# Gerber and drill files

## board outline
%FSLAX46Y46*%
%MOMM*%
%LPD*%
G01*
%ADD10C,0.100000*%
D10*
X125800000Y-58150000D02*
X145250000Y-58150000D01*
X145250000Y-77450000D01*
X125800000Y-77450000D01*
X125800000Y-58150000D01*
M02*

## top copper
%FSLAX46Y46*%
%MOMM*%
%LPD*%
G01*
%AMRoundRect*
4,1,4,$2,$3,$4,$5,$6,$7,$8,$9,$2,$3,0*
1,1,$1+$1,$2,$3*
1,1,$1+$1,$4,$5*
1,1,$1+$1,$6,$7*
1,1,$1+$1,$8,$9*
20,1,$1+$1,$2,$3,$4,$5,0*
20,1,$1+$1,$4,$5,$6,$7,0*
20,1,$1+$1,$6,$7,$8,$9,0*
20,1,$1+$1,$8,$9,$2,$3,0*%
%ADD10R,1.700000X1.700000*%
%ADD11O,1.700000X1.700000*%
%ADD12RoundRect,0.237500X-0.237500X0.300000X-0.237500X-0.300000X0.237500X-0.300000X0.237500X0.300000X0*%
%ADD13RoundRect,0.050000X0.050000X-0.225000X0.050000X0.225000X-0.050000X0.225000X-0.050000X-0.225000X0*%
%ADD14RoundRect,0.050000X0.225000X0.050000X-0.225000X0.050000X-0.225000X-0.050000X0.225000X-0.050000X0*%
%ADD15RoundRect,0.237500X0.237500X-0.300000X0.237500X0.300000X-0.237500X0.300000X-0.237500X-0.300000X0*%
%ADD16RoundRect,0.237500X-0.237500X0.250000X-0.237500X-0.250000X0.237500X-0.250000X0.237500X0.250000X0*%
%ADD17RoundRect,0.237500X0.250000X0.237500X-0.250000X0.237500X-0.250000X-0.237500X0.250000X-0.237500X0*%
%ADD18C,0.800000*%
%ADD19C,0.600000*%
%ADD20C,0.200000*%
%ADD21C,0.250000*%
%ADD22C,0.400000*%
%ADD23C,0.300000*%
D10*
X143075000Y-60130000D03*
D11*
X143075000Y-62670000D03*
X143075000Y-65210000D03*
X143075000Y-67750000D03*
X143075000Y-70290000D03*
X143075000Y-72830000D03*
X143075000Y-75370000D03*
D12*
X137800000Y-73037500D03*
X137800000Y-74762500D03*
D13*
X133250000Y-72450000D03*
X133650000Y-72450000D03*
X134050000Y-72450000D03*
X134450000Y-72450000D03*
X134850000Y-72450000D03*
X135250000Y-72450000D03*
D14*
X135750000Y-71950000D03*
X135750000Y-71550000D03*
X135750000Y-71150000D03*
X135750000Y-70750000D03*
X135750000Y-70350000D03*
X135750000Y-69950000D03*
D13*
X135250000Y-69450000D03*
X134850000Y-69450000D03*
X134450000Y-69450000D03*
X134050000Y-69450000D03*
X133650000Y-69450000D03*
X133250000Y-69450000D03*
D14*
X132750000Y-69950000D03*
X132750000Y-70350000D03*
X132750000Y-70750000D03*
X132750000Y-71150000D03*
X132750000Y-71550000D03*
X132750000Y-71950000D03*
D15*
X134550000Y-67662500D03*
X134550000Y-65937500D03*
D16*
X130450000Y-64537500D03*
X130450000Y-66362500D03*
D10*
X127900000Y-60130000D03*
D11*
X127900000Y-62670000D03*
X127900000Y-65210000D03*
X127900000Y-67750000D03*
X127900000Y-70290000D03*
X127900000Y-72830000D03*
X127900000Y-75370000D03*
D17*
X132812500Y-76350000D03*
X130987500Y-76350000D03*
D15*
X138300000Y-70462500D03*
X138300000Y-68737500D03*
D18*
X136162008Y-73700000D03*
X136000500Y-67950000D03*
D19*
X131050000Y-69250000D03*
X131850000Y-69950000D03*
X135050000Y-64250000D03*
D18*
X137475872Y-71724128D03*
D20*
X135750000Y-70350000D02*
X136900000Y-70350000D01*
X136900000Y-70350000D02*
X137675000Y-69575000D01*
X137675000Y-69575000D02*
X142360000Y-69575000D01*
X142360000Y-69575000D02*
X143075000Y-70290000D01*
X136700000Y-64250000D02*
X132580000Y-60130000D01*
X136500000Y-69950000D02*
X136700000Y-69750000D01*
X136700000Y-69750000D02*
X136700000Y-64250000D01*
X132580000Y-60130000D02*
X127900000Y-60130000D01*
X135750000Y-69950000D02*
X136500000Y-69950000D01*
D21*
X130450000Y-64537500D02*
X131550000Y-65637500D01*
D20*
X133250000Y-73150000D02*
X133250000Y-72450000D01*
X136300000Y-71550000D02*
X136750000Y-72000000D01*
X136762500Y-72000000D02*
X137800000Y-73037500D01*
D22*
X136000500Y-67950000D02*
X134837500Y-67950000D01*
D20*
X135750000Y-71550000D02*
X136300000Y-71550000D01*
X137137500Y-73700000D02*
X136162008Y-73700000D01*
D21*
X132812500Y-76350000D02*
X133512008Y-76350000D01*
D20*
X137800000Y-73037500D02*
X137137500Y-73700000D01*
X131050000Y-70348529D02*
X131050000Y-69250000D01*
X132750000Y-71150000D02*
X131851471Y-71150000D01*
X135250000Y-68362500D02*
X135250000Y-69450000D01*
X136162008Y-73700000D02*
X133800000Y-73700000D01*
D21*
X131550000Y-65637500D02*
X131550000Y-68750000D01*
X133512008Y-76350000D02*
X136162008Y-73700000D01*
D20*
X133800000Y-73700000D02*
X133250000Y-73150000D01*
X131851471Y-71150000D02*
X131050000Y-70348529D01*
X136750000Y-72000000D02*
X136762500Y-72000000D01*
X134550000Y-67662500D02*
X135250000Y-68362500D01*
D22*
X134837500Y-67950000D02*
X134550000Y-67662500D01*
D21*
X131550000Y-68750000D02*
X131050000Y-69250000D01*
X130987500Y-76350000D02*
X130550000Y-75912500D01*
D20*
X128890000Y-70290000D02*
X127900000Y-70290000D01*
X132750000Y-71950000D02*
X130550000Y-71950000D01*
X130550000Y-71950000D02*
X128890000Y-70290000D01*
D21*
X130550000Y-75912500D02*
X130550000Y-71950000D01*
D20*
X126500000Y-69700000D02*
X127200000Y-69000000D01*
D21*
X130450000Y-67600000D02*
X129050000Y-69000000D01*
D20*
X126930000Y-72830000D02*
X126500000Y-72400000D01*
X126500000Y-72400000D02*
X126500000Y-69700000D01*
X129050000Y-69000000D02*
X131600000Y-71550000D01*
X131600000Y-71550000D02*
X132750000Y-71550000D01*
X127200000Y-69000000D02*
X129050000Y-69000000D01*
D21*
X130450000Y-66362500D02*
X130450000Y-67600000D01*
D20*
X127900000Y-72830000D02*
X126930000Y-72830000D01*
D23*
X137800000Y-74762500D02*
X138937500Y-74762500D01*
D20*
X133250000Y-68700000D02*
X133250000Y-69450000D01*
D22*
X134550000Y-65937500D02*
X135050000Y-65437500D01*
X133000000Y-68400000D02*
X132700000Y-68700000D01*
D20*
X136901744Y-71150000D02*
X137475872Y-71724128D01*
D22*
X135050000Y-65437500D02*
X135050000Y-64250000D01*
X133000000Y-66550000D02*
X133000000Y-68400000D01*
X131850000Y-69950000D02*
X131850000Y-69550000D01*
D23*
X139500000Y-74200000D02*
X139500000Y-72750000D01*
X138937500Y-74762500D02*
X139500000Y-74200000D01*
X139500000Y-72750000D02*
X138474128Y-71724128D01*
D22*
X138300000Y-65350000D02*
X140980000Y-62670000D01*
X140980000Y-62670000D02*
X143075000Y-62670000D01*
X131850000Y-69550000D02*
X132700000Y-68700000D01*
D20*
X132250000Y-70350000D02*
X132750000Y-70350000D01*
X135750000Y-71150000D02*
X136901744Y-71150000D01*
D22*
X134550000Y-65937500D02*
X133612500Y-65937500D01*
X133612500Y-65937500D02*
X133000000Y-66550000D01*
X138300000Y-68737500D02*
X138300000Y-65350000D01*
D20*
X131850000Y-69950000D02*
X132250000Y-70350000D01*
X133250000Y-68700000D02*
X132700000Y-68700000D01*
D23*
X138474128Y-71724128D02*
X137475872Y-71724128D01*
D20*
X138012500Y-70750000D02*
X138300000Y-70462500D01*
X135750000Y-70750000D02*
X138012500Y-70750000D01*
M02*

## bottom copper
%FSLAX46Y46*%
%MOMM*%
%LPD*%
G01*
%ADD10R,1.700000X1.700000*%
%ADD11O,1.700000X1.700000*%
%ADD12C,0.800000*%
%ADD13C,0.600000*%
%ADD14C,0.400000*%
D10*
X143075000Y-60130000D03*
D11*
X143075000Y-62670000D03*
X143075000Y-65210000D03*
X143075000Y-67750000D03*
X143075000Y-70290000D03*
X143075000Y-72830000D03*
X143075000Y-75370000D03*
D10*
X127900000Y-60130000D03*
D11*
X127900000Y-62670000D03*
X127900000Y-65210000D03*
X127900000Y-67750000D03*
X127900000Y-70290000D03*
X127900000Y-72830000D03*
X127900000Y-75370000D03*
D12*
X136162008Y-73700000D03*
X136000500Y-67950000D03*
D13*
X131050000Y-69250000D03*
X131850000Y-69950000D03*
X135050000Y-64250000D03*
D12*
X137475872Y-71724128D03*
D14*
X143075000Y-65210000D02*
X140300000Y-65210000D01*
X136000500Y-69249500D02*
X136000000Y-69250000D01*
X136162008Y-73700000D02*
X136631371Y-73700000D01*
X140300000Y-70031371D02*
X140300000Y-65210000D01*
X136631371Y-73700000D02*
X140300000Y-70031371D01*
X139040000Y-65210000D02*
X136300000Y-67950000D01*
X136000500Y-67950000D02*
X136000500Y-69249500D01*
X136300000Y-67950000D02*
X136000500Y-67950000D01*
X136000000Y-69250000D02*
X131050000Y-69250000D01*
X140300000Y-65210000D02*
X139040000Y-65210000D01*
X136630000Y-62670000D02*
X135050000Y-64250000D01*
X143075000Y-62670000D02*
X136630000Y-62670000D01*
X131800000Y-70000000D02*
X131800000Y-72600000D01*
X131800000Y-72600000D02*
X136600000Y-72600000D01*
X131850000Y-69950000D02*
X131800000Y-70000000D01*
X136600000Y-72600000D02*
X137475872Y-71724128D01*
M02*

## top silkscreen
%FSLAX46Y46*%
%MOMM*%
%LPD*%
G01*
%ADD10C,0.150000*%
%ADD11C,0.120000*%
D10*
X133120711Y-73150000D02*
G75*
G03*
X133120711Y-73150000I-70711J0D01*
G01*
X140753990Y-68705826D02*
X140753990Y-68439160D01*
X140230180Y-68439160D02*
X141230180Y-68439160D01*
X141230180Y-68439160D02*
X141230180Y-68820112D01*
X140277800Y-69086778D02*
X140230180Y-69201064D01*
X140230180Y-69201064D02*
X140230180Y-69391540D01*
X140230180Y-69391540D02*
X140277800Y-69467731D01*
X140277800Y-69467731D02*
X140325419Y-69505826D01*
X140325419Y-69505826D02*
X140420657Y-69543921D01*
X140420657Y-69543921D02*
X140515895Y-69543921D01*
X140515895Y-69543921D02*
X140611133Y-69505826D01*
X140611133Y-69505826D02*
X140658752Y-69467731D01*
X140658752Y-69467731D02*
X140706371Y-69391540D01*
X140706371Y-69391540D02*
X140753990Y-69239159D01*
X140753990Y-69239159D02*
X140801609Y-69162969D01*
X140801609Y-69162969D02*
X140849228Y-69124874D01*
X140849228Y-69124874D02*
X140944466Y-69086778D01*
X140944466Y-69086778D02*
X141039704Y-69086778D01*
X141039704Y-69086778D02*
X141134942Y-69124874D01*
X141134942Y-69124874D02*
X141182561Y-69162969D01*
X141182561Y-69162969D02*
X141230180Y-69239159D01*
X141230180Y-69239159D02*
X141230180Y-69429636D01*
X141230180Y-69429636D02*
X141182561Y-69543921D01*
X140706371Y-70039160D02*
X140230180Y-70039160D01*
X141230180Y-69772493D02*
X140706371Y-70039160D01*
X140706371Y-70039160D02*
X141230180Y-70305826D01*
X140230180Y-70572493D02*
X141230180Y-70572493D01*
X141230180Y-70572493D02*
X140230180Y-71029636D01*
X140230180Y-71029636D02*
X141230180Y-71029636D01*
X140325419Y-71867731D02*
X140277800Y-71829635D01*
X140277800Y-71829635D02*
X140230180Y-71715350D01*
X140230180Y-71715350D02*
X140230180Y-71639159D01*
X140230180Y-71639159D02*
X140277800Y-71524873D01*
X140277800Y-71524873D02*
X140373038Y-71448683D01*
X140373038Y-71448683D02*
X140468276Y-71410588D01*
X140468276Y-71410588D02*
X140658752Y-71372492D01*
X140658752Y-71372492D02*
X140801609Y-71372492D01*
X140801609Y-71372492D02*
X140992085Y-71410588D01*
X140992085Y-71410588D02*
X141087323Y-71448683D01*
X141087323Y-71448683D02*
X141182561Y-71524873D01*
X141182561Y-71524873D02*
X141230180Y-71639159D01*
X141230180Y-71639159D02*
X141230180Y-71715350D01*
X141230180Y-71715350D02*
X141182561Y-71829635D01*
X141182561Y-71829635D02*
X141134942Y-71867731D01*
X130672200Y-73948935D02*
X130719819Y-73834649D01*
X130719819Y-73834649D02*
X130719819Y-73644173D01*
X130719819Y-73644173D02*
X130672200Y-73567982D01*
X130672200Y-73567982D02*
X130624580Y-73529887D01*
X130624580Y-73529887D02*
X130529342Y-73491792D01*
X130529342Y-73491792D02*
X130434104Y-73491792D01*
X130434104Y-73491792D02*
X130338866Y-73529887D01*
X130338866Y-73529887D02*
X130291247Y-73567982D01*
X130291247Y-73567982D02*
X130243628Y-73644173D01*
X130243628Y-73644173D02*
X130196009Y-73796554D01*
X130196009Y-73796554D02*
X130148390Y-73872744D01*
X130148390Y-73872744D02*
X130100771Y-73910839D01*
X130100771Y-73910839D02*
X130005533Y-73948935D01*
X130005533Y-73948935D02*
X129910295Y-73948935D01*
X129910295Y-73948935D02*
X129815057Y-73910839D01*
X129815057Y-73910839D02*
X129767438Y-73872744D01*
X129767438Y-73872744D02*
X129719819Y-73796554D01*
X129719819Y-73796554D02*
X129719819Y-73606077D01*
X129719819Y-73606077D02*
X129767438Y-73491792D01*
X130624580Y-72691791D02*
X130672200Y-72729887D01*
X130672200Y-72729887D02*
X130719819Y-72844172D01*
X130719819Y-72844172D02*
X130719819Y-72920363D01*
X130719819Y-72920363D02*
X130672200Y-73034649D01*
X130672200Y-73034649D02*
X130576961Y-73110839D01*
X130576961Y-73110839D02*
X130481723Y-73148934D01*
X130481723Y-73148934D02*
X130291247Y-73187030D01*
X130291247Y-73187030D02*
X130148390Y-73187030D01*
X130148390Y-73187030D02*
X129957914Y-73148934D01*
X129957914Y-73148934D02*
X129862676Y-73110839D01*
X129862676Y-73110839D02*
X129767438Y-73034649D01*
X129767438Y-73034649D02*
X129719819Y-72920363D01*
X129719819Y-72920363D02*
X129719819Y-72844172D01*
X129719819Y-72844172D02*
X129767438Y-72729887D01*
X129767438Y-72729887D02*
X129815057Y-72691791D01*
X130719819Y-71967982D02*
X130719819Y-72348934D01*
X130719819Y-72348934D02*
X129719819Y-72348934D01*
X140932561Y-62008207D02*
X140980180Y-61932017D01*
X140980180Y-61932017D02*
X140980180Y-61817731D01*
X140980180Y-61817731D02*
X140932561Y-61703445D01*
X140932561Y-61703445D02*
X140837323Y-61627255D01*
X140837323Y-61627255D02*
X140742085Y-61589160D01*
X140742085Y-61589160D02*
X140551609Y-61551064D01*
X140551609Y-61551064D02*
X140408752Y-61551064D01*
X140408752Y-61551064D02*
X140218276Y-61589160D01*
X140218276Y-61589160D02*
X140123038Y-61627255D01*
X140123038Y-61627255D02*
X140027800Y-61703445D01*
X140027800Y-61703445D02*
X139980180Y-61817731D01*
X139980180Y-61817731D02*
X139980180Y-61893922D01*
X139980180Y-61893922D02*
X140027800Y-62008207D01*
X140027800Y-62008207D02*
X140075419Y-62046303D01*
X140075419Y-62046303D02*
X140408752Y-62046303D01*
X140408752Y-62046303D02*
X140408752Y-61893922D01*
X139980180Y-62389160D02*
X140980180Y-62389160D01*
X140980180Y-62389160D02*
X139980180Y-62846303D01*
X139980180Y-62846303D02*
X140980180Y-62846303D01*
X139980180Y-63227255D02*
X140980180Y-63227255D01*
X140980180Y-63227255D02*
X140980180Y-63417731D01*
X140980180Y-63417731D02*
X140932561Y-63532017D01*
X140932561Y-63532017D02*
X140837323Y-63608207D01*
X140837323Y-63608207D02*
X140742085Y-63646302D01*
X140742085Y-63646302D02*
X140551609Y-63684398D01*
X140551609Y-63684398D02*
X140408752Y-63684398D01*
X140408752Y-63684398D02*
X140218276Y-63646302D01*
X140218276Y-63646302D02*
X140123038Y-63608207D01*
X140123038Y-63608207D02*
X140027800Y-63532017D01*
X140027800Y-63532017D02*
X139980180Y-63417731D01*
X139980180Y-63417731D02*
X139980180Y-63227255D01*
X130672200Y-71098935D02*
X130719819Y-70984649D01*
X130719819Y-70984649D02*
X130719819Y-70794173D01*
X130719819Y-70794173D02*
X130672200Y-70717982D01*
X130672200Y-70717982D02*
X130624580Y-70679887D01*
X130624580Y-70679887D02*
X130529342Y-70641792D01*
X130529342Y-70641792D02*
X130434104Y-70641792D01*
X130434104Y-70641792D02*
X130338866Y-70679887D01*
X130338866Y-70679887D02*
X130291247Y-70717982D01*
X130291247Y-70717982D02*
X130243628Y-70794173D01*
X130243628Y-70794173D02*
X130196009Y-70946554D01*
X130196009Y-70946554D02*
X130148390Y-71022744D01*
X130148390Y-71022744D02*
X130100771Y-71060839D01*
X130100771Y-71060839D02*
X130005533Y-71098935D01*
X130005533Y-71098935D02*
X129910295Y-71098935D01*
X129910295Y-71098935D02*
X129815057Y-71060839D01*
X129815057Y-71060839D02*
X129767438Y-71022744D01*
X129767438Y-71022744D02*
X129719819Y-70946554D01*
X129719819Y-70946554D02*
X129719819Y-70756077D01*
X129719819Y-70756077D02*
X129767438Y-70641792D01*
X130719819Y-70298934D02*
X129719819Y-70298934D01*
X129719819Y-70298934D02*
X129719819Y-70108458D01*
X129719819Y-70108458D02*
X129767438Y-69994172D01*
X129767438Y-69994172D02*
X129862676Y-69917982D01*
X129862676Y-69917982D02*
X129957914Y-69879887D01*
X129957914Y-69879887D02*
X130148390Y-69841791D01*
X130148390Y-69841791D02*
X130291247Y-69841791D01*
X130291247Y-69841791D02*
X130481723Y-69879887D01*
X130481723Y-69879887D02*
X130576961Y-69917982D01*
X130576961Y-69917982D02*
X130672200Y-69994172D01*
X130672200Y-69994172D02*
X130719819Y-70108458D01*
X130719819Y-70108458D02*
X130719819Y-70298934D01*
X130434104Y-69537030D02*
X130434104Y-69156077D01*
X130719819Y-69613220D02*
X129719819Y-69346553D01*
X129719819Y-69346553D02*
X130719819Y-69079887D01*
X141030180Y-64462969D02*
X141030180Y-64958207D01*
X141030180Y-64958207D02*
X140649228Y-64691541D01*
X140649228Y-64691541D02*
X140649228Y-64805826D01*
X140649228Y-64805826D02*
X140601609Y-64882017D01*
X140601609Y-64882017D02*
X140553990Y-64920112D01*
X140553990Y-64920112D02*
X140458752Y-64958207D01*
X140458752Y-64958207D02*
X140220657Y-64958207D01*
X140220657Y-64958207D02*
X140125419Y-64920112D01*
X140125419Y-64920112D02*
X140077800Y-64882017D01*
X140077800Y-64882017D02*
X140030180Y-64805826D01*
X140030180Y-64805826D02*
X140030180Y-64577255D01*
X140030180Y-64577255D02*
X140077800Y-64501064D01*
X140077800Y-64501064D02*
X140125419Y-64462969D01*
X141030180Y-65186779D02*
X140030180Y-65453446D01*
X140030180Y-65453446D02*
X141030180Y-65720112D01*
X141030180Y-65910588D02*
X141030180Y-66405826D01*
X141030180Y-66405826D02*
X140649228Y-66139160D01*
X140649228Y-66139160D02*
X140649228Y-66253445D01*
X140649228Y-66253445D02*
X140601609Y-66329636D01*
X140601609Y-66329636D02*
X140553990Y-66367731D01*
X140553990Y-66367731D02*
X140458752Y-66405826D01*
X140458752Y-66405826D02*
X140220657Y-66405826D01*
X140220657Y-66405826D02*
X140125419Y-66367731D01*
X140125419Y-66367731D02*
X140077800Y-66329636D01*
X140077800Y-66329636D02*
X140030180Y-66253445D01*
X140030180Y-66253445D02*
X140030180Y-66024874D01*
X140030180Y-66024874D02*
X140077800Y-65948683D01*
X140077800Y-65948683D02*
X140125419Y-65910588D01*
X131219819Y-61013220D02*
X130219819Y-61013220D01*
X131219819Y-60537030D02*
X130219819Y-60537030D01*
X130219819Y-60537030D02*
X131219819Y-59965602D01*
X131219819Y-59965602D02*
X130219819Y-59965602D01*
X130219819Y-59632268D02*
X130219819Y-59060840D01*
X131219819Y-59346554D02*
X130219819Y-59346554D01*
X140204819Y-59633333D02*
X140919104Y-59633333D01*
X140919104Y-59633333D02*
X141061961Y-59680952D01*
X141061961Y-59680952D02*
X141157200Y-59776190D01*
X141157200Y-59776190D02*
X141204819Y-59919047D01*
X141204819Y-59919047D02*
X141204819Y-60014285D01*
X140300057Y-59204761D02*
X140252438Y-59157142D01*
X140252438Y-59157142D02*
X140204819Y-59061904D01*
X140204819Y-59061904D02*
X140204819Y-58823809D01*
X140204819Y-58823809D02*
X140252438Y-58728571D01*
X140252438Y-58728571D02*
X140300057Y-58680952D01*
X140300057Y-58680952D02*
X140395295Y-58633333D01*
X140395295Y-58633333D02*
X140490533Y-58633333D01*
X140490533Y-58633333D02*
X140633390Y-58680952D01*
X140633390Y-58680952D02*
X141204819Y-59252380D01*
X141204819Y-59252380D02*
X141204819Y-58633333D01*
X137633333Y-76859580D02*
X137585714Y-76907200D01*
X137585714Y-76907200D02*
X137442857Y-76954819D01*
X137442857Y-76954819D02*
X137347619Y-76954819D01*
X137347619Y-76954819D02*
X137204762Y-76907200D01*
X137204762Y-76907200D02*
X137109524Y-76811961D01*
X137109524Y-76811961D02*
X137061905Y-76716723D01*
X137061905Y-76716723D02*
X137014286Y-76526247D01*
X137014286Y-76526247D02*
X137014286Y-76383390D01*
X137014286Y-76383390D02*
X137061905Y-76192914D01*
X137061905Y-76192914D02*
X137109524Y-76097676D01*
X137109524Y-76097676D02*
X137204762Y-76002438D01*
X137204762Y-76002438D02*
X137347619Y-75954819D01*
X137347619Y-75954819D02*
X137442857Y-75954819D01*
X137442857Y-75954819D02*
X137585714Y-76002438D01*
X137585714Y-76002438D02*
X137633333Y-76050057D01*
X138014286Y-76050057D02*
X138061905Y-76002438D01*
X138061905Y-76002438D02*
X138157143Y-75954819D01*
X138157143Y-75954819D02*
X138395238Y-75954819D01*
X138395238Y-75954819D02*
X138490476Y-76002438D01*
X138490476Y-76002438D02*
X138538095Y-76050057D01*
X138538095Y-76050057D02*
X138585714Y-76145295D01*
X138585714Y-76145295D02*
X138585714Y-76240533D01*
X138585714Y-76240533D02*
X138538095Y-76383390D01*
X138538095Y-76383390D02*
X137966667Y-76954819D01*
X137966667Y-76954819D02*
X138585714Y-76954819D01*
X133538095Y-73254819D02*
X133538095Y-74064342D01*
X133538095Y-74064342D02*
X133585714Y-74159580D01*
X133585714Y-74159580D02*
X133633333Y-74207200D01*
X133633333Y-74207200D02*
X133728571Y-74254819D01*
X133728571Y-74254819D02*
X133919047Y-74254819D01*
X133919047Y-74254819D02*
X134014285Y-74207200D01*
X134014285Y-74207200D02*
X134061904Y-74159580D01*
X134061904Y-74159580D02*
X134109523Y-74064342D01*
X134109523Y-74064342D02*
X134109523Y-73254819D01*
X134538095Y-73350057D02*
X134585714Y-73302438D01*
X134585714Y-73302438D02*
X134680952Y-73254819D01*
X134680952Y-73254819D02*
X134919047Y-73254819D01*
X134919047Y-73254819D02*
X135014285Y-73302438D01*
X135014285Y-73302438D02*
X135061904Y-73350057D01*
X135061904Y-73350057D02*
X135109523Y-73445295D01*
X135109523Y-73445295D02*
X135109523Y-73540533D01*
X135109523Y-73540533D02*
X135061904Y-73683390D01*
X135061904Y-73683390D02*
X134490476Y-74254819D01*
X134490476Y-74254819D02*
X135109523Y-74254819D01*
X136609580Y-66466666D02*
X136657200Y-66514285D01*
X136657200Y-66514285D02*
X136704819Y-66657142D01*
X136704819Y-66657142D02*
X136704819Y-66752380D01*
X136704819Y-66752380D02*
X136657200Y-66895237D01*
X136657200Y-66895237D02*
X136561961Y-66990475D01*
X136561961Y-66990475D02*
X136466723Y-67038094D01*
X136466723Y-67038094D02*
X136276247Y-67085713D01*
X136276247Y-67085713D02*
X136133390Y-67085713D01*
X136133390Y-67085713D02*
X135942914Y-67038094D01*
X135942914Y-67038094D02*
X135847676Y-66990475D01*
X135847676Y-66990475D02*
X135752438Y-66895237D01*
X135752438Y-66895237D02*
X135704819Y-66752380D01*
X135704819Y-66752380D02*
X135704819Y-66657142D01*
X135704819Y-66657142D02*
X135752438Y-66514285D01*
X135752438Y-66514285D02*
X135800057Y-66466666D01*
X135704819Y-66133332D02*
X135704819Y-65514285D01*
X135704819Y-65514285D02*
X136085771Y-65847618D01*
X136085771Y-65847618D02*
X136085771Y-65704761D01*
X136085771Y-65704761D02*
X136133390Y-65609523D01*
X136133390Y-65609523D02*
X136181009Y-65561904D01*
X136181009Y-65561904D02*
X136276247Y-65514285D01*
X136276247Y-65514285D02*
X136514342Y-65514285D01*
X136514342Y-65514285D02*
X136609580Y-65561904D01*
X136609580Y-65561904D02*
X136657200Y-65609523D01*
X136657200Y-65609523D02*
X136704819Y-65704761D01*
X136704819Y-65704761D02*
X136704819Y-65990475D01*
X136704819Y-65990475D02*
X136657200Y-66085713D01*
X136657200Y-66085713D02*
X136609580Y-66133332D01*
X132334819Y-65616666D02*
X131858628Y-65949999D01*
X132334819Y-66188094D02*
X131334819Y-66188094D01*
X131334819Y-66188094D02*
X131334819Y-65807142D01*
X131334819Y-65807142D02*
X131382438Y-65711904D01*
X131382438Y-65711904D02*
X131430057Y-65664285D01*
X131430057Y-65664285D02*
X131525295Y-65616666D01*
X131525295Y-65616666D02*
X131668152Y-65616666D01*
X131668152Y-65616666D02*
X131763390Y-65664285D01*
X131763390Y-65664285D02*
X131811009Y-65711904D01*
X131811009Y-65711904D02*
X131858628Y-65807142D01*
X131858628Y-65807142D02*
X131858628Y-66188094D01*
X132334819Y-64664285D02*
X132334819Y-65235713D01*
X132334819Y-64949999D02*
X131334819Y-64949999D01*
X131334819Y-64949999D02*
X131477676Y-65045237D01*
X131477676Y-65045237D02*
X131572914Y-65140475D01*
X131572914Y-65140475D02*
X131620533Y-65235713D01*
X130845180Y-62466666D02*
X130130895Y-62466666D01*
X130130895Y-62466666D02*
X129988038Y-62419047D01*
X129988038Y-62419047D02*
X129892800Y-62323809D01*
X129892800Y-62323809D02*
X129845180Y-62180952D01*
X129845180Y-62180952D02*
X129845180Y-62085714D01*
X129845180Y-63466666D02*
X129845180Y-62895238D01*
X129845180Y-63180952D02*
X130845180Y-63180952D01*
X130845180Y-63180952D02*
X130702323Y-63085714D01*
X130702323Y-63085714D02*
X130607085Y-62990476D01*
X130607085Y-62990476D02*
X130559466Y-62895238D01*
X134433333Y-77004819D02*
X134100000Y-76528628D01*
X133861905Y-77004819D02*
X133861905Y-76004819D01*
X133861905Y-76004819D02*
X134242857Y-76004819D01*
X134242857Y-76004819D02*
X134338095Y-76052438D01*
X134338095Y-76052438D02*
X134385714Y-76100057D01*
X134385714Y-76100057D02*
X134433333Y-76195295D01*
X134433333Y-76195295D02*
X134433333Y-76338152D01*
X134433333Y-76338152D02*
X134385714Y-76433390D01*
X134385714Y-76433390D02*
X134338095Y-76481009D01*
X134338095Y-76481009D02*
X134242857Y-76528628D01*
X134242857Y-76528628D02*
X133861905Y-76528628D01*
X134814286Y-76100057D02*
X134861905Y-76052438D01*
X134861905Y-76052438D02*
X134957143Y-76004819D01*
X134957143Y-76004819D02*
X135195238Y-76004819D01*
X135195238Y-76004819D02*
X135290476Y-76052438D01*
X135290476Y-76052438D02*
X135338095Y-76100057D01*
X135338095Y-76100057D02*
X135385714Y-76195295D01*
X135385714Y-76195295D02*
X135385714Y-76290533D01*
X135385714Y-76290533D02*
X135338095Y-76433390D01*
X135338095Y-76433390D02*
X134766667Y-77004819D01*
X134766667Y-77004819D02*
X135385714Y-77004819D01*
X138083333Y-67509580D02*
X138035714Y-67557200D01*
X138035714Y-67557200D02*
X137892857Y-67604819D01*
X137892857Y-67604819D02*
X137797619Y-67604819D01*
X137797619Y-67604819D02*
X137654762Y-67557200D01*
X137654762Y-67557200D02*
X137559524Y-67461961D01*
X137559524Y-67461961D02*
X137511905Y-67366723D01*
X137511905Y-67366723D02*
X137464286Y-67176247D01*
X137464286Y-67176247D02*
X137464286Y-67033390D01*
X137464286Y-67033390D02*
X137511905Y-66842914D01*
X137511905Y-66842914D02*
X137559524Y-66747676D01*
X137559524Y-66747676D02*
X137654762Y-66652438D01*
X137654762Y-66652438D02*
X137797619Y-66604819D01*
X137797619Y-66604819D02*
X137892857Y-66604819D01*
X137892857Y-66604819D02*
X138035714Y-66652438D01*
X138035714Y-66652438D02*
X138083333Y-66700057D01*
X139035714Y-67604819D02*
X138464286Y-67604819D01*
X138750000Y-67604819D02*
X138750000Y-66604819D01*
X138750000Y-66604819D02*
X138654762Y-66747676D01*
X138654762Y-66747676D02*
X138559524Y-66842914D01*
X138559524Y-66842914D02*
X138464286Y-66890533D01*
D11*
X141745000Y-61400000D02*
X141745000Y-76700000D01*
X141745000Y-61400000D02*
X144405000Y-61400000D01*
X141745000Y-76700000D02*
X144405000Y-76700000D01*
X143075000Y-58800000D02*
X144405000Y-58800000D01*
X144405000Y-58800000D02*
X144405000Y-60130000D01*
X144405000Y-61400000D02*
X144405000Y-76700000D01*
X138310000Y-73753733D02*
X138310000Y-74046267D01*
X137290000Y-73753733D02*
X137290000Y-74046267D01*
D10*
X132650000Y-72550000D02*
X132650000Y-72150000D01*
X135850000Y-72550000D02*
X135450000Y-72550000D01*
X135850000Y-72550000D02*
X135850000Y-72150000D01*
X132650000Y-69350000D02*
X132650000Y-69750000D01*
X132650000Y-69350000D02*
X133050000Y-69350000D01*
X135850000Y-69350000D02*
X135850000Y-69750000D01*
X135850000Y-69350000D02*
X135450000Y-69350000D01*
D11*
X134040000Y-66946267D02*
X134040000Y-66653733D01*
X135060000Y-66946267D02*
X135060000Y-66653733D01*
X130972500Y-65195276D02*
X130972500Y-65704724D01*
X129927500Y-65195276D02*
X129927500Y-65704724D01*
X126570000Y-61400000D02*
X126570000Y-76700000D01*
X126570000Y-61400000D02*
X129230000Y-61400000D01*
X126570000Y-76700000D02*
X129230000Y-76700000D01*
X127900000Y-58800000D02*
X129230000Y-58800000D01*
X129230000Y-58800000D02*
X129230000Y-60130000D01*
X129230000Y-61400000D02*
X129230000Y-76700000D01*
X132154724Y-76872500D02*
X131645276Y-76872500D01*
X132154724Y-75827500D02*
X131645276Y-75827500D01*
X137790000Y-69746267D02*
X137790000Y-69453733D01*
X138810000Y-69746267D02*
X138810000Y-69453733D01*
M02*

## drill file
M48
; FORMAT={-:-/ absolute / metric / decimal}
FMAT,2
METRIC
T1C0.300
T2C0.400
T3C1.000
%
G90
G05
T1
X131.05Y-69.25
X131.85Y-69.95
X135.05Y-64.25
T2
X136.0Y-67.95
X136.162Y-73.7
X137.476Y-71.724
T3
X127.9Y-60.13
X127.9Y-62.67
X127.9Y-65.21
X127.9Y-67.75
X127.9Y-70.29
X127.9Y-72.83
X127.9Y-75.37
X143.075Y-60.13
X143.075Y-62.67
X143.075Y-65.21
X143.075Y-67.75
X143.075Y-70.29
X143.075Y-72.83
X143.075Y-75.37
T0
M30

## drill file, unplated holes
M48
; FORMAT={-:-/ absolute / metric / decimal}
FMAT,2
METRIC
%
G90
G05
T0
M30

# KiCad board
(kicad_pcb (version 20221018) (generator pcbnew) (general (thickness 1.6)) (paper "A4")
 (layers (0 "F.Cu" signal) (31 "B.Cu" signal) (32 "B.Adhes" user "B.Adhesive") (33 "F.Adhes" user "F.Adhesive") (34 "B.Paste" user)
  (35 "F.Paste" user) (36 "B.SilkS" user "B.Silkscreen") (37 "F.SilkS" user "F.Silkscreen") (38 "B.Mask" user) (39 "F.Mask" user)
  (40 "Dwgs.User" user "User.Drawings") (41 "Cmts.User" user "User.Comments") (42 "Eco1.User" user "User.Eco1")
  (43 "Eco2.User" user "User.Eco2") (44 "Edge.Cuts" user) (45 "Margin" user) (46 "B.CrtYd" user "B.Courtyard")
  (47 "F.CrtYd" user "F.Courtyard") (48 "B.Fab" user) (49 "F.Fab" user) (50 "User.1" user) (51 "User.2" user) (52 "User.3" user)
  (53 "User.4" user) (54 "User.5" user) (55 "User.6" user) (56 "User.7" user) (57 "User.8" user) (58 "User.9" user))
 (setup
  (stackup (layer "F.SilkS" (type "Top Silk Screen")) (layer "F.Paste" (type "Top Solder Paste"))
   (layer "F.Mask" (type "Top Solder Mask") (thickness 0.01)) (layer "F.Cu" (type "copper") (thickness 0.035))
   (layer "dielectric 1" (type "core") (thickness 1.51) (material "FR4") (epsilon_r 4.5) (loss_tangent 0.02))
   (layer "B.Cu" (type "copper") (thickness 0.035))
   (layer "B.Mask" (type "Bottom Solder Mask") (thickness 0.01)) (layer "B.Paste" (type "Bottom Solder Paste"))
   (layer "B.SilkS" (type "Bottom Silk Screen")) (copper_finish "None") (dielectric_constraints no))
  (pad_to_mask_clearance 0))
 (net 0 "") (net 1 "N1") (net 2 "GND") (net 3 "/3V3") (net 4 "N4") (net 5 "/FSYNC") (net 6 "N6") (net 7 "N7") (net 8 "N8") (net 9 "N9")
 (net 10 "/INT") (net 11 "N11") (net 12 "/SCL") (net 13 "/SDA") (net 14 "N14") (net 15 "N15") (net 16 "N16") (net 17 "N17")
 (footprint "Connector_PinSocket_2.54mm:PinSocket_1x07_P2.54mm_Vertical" (layer "F.Cu") (at 143.075 60.13)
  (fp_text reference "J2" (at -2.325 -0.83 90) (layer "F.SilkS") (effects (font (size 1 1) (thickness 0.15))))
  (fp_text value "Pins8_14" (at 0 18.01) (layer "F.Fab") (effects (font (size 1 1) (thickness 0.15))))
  (fp_line (start -1.33 1.27) (end -1.33 16.57) (stroke (width 0.12) (type solid)) (layer "F.SilkS"))
  (fp_line (start -1.33 1.27) (end 1.33 1.27) (stroke (width 0.12) (type solid)) (layer "F.SilkS"))
  (fp_line (start -1.33 16.57) (end 1.33 16.57) (stroke (width 0.12) (type solid)) (layer "F.SilkS"))
  (fp_line (start 0 -1.33) (end 1.33 -1.33) (stroke (width 0.12) (type solid)) (layer "F.SilkS"))
  (fp_line (start 1.33 -1.33) (end 1.33 0) (stroke (width 0.12) (type solid)) (layer "F.SilkS"))
  (fp_line (start 1.33 1.27) (end 1.33 16.57) (stroke (width 0.12) (type solid)) (layer "F.SilkS"))
  (pad "1" thru_hole rect (at 0 0) (size 1.7 1.7) (drill 1) (layers "*.Cu" "*.Mask") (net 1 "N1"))
  (pad "2" thru_hole oval (at 0 2.54) (size 1.7 1.7) (drill 1) (layers "*.Cu" "*.Mask") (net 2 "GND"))
  (pad "3" thru_hole oval (at 0 5.08) (size 1.7 1.7) (drill 1) (layers "*.Cu" "*.Mask") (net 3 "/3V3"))
  (pad "4" thru_hole oval (at 0 7.62) (size 1.7 1.7) (drill 1) (layers "*.Cu" "*.Mask") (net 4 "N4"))
  (pad "5" thru_hole oval (at 0 10.16) (size 1.7 1.7) (drill 1) (layers "*.Cu" "*.Mask") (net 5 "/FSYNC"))
  (pad "6" thru_hole oval (at 0 12.7) (size 1.7 1.7) (drill 1) (layers "*.Cu" "*.Mask") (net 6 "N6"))
  (pad "7" thru_hole oval (at 0 15.24) (size 1.7 1.7) (drill 1) (layers "*.Cu" "*.Mask") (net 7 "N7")))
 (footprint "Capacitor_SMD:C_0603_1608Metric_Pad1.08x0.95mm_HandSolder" (layer "F.Cu") (at 137.8 73.9 -90)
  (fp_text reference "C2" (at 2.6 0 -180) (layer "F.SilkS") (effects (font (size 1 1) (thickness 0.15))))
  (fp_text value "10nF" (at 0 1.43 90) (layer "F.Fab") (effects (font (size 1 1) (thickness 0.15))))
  (fp_line (start -0.146267 -0.51) (end 0.146267 -0.51) (stroke (width 0.12) (type solid)) (layer "F.SilkS"))
  (fp_line (start -0.146267 0.51) (end 0.146267 0.51) (stroke (width 0.12) (type solid)) (layer "F.SilkS"))
  (pad "1" smd roundrect (at -0.8625 0 270) (size 1.075 0.95) (layers "F.Cu" "F.Paste" "F.Mask") (roundrect_rratio 0.25) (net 3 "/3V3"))
  (pad "2" smd roundrect (at 0.8625 0 270) (size 1.075 0.95) (layers "F.Cu" "F.Paste" "F.Mask") (roundrect_rratio 0.25) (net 2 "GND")))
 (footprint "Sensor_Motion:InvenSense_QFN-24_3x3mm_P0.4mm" (layer "F.Cu") (at 134.25 70.95 90)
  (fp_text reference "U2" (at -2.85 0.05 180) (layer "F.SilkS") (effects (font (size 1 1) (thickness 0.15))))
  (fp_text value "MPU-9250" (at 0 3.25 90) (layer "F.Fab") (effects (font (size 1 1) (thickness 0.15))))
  (fp_line (start -1.6 -1.6) (end -1.2 -1.6) (stroke (width 0.15) (type solid)) (layer "F.SilkS"))
  (fp_line (start -1.6 1.6) (end -1.6 1.2) (stroke (width 0.15) (type solid)) (layer "F.SilkS"))
  (fp_line (start -1.6 1.6) (end -1.2 1.6) (stroke (width 0.15) (type solid)) (layer "F.SilkS"))
  (fp_line (start 1.6 -1.6) (end 1.2 -1.6) (stroke (width 0.15) (type solid)) (layer "F.SilkS"))
  (fp_line (start 1.6 -1.6) (end 1.6 -1.2) (stroke (width 0.15) (type solid)) (layer "F.SilkS"))
  (fp_line (start 1.6 1.6) (end 1.2 1.6) (stroke (width 0.15) (type solid)) (layer "F.SilkS"))
  (fp_line (start 1.6 1.6) (end 1.6 1.2) (stroke (width 0.15) (type solid)) (layer "F.SilkS"))
  (pad "1" smd roundrect (at -1.5 -1 90) (size 0.55 0.2) (layers "F.Cu" "F.Paste" "F.Mask") (roundrect_rratio 0.25) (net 3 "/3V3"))
  (pad "2" smd roundrect (at -1.5 -0.6 90) (size 0.55 0.2) (layers "F.Cu" "F.Paste" "F.Mask") (roundrect_rratio 0.25))
  (pad "3" smd roundrect (at -1.5 -0.2 90) (size 0.55 0.2) (layers "F.Cu" "F.Paste" "F.Mask") (roundrect_rratio 0.25))
  (pad "4" smd roundrect (at -1.5 0.2 90) (size 0.55 0.2) (layers "F.Cu" "F.Paste" "F.Mask") (roundrect_rratio 0.25))
  (pad "5" smd roundrect (at -1.5 0.6 90) (size 0.55 0.2) (layers "F.Cu" "F.Paste" "F.Mask") (roundrect_rratio 0.25))
  (pad "6" smd roundrect (at -1.5 1 90) (size 0.55 0.2) (layers "F.Cu" "F.Paste" "F.Mask") (roundrect_rratio 0.25))
  (pad "7" smd roundrect (at -1 1.5 180) (size 0.55 0.2) (layers "F.Cu" "F.Paste" "F.Mask") (roundrect_rratio 0.25) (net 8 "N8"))
  (pad "8" smd roundrect (at -0.6 1.5 180) (size 0.55 0.2) (layers "F.Cu" "F.Paste" "F.Mask") (roundrect_rratio 0.25) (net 3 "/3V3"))
  (pad "9" smd roundrect (at -0.2 1.5 180) (size 0.55 0.2) (layers "F.Cu" "F.Paste" "F.Mask") (roundrect_rratio 0.25) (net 2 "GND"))
  (pad "10" smd roundrect (at 0.2 1.5 180) (size 0.55 0.2) (layers "F.Cu" "F.Paste" "F.Mask") (roundrect_rratio 0.25) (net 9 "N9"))
  (pad "11" smd roundrect (at 0.6 1.5 180) (size 0.55 0.2) (layers "F.Cu" "F.Paste" "F.Mask") (roundrect_rratio 0.25) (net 5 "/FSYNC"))
  (pad "12" smd roundrect (at 1 1.5 180) (size 0.55 0.2) (layers "F.Cu" "F.Paste" "F.Mask") (roundrect_rratio 0.25) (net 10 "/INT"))
  (pad "13" smd roundrect (at 1.5 1 90) (size 0.55 0.2) (layers "F.Cu" "F.Paste" "F.Mask") (roundrect_rratio 0.25) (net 3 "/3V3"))
  (pad "14" smd roundrect (at 1.5 0.6 90) (size 0.55 0.2) (layers "F.Cu" "F.Paste" "F.Mask") (roundrect_rratio 0.25))
  (pad "15" smd roundrect (at 1.5 0.2 90) (size 0.55 0.2) (layers "F.Cu" "F.Paste" "F.Mask") (roundrect_rratio 0.25))
  (pad "16" smd roundrect (at 1.5 -0.2 90) (size 0.55 0.2) (layers "F.Cu" "F.Paste" "F.Mask") (roundrect_rratio 0.25))
  (pad "17" smd roundrect (at 1.5 -0.6 90) (size 0.55 0.2) (layers "F.Cu" "F.Paste" "F.Mask") (roundrect_rratio 0.25))
  (pad "18" smd roundrect (at 1.5 -1 90) (size 0.55 0.2) (layers "F.Cu" "F.Paste" "F.Mask") (roundrect_rratio 0.25) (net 2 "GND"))
  (pad "19" smd roundrect (at 1 -1.5 180) (size 0.55 0.2) (layers "F.Cu" "F.Paste" "F.Mask") (roundrect_rratio 0.25))
  (pad "20" smd roundrect (at 0.6 -1.5 180) (size 0.55 0.2) (layers "F.Cu" "F.Paste" "F.Mask") (roundrect_rratio 0.25) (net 2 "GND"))
  (pad "21" smd roundrect (at 0.2 -1.5 180) (size 0.55 0.2) (layers "F.Cu" "F.Paste" "F.Mask") (roundrect_rratio 0.25) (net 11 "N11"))
  (pad "22" smd roundrect (at -0.2 -1.5 180) (size 0.55 0.2) (layers "F.Cu" "F.Paste" "F.Mask") (roundrect_rratio 0.25) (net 3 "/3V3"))
  (pad "23" smd roundrect (at -0.6 -1.5 180) (size 0.55 0.2) (layers "F.Cu" "F.Paste" "F.Mask") (roundrect_rratio 0.25) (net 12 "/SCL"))
  (pad "24" smd roundrect (at -1 -1.5 180) (size 0.55 0.2) (layers "F.Cu" "F.Paste" "F.Mask") (roundrect_rratio 0.25) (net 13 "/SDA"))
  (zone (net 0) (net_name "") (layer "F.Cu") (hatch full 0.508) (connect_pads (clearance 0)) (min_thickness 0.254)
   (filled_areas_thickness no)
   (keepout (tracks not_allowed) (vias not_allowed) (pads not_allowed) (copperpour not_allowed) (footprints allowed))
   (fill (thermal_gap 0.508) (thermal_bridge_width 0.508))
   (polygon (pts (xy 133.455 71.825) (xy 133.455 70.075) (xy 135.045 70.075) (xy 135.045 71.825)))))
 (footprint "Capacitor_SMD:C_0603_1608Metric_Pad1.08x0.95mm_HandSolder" (layer "F.Cu") (at 134.55 66.8 90)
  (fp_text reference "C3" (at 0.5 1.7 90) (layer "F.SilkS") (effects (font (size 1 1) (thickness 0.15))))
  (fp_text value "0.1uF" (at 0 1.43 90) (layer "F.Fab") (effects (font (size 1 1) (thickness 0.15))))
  (fp_line (start -0.146267 -0.51) (end 0.146267 -0.51) (stroke (width 0.12) (type solid)) (layer "F.SilkS"))
  (fp_line (start -0.146267 0.51) (end 0.146267 0.51) (stroke (width 0.12) (type solid)) (layer "F.SilkS"))
  (pad "1" smd roundrect (at -0.8625 0 90) (size 1.075 0.95) (layers "F.Cu" "F.Paste" "F.Mask") (roundrect_rratio 0.25) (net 3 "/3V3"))
  (pad "2" smd roundrect (at 0.8625 0 90) (size 1.075 0.95) (layers "F.Cu" "F.Paste" "F.Mask") (roundrect_rratio 0.25) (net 2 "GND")))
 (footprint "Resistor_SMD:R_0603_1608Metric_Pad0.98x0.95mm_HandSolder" (layer "F.Cu") (at 130.45 65.45 -90)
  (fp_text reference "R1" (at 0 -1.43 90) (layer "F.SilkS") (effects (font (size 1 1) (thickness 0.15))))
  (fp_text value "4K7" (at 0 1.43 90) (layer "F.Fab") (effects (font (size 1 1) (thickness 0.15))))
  (fp_line (start -0.254724 -0.5225) (end 0.254724 -0.5225) (stroke (width 0.12) (type solid)) (layer "F.SilkS"))
  (fp_line (start -0.254724 0.5225) (end 0.254724 0.5225) (stroke (width 0.12) (type solid)) (layer "F.SilkS"))
  (pad "1" smd roundrect (at -0.9125 0 270) (size 0.975 0.95) (layers "F.Cu" "F.Paste" "F.Mask") (roundrect_rratio 0.25) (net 3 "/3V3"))
  (pad "2" smd roundrect (at 0.9125 0 270) (size 0.975 0.95) (layers "F.Cu" "F.Paste" "F.Mask") (roundrect_rratio 0.25) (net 12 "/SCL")))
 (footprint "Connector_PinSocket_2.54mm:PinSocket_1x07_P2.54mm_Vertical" (layer "F.Cu") (at 127.9 60.13)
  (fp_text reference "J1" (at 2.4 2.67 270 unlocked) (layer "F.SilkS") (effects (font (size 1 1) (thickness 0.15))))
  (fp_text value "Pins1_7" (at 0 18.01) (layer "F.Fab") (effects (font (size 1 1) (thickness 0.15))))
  (fp_line (start -1.33 1.27) (end -1.33 16.57) (stroke (width 0.12) (type solid)) (layer "F.SilkS"))
  (fp_line (start -1.33 1.27) (end 1.33 1.27) (stroke (width 0.12) (type solid)) (layer "F.SilkS"))
  (fp_line (start -1.33 16.57) (end 1.33 16.57) (stroke (width 0.12) (type solid)) (layer "F.SilkS"))
  (fp_line (start 0 -1.33) (end 1.33 -1.33) (stroke (width 0.12) (type solid)) (layer "F.SilkS"))
  (fp_line (start 1.33 -1.33) (end 1.33 0) (stroke (width 0.12) (type solid)) (layer "F.SilkS"))
  (fp_line (start 1.33 1.27) (end 1.33 16.57) (stroke (width 0.12) (type solid)) (layer "F.SilkS"))
  (pad "1" thru_hole rect (at 0 0) (size 1.7 1.7) (drill 1) (layers "*.Cu" "*.Mask") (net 10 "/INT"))
  (pad "2" thru_hole oval (at 0 2.54) (size 1.7 1.7) (drill 1) (layers "*.Cu" "*.Mask") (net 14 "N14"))
  (pad "3" thru_hole oval (at 0 5.08) (size 1.7 1.7) (drill 1) (layers "*.Cu" "*.Mask") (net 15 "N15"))
  (pad "4" thru_hole oval (at 0 7.62) (size 1.7 1.7) (drill 1) (layers "*.Cu" "*.Mask") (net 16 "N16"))
  (pad "5" thru_hole oval (at 0 10.16) (size 1.7 1.7) (drill 1) (layers "*.Cu" "*.Mask") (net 13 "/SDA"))
  (pad "6" thru_hole oval (at 0 12.7) (size 1.7 1.7) (drill 1) (layers "*.Cu" "*.Mask") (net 12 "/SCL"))
  (pad "7" thru_hole oval (at 0 15.24) (size 1.7 1.7) (drill 1) (layers "*.Cu" "*.Mask") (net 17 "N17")))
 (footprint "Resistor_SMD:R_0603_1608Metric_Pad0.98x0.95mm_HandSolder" (layer "F.Cu") (at 131.9 76.35 180)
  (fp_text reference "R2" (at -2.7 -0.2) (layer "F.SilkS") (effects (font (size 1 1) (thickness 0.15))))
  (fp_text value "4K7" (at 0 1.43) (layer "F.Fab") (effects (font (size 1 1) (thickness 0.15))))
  (fp_line (start -0.254724 -0.5225) (end 0.254724 -0.5225) (stroke (width 0.12) (type solid)) (layer "F.SilkS"))
  (fp_line (start -0.254724 0.5225) (end 0.254724 0.5225) (stroke (width 0.12) (type solid)) (layer "F.SilkS"))
  (pad "1" smd roundrect (at -0.9125 0 180) (size 0.975 0.95) (layers "F.Cu" "F.Paste" "F.Mask") (roundrect_rratio 0.25) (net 3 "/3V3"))
  (pad "2" smd roundrect (at 0.9125 0 180) (size 0.975 0.95) (layers "F.Cu" "F.Paste" "F.Mask") (roundrect_rratio 0.25) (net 13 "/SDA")))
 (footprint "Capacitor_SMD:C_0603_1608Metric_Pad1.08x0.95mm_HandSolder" (layer "F.Cu") (at 138.3 69.6 90)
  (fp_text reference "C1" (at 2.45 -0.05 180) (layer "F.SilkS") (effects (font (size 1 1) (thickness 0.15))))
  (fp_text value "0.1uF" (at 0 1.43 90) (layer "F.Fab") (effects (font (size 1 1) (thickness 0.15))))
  (fp_line (start -0.146267 -0.51) (end 0.146267 -0.51) (stroke (width 0.12) (type solid)) (layer "F.SilkS"))
  (fp_line (start -0.146267 0.51) (end 0.146267 0.51) (stroke (width 0.12) (type solid)) (layer "F.SilkS"))
  (pad "1" smd roundrect (at -0.8625 0 90) (size 1.075 0.95) (layers "F.Cu" "F.Paste" "F.Mask") (roundrect_rratio 0.25) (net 9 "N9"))
  (pad "2" smd roundrect (at 0.8625 0 90) (size 1.075 0.95) (layers "F.Cu" "F.Paste" "F.Mask") (roundrect_rratio 0.25) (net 2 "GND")))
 (gr_circle (center 133.05 73.15) (end 133.1 73.2) (stroke (width 0.15) (type default)) (fill none) (layer "F.SilkS"))
 (gr_rect (start 125.8 58.15) (end 145.25 77.45) (stroke (width 0.1) (type default)) (fill none) (layer "Edge.Cuts"))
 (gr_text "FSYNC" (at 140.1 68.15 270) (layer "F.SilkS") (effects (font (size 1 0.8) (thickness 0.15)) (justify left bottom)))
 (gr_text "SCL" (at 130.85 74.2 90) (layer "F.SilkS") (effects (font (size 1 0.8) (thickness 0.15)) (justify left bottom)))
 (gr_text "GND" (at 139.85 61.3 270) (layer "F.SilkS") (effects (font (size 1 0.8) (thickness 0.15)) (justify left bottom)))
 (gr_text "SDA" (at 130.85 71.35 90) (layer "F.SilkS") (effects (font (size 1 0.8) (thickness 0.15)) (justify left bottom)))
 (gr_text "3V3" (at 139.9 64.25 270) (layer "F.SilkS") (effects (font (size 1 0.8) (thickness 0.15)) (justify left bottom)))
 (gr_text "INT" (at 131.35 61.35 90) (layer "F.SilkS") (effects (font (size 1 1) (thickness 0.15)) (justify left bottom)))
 (segment (start 135.75 70.35) (end 136.9 70.35) (width 0.2) (layer "F.Cu") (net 5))
 (segment (start 136.9 70.35) (end 137.675 69.575) (width 0.2) (layer "F.Cu") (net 5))
 (segment (start 137.675 69.575) (end 142.36 69.575) (width 0.2) (layer "F.Cu") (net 5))
 (segment (start 142.36 69.575) (end 143.075 70.29) (width 0.2) (layer "F.Cu") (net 5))
 (segment (start 136.7 64.25) (end 132.58 60.13) (width 0.2) (layer "F.Cu") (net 10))
 (segment (start 136.5 69.95) (end 136.7 69.75) (width 0.2) (layer "F.Cu") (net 10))
 (segment (start 136.7 69.75) (end 136.7 64.25) (width 0.2) (layer "F.Cu") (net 10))
 (segment (start 132.58 60.13) (end 127.9 60.13) (width 0.2) (layer "F.Cu") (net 10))
 (segment (start 135.75 69.95) (end 136.5 69.95) (width 0.2) (layer "F.Cu") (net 10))
 (segment (start 130.45 64.5375) (end 131.55 65.6375) (width 0.25) (layer "F.Cu") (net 3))
 (segment (start 133.25 73.15) (end 133.25 72.45) (width 0.2) (layer "F.Cu") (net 3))
 (segment (start 136.3 71.55) (end 136.75 72) (width 0.2) (layer "F.Cu") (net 3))
 (segment (start 136.7625 72) (end 137.8 73.0375) (width 0.2) (layer "F.Cu") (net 3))
 (segment (start 136.0005 67.95) (end 134.8375 67.95) (width 0.4) (layer "F.Cu") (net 3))
 (segment (start 135.75 71.55) (end 136.3 71.55) (width 0.2) (layer "F.Cu") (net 3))
 (segment (start 137.1375 73.7) (end 136.162008 73.7) (width 0.2) (layer "F.Cu") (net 3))
 (segment (start 132.8125 76.35) (end 133.512008 76.35) (width 0.25) (layer "F.Cu") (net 3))
 (segment (start 137.8 73.0375) (end 137.1375 73.7) (width 0.2) (layer "F.Cu") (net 3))
 (segment (start 131.05 70.348529) (end 131.05 69.25) (width 0.2) (layer "F.Cu") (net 3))
 (segment (start 132.75 71.15) (end 131.851471 71.15) (width 0.2) (layer "F.Cu") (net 3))
 (segment (start 135.25 68.3625) (end 135.25 69.45) (width 0.2) (layer "F.Cu") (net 3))
 (segment (start 136.162008 73.7) (end 133.8 73.7) (width 0.2) (layer "F.Cu") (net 3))
 (segment (start 131.55 65.6375) (end 131.55 68.75) (width 0.25) (layer "F.Cu") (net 3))
 (segment (start 133.512008 76.35) (end 136.162008 73.7) (width 0.25) (layer "F.Cu") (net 3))
 (segment (start 133.8 73.7) (end 133.25 73.15) (width 0.2) (layer "F.Cu") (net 3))
 (segment (start 131.851471 71.15) (end 131.05 70.348529) (width 0.2) (layer "F.Cu") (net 3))
 (segment (start 136.75 72) (end 136.7625 72) (width 0.2) (layer "F.Cu") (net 3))
 (segment (start 134.55 67.6625) (end 135.25 68.3625) (width 0.2) (layer "F.Cu") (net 3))
 (segment (start 134.8375 67.95) (end 134.55 67.6625) (width 0.4) (layer "F.Cu") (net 3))
 (segment (start 131.55 68.75) (end 131.05 69.25) (width 0.25) (layer "F.Cu") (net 3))
 (via (at 136.162008 73.7) (size 0.8) (drill 0.4) (layers "F.Cu" "B.Cu") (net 3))
 (via (at 136.0005 67.95) (size 0.8) (drill 0.4) (layers "F.Cu" "B.Cu") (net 3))
 (via (at 131.05 69.25) (size 0.6) (drill 0.3) (layers "F.Cu" "B.Cu") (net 3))
 (segment (start 143.075 65.21) (end 140.3 65.21) (width 0.4) (layer "B.Cu") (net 3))
 (segment (start 136.0005 69.2495) (end 136 69.25) (width 0.4) (layer "B.Cu") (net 3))
 (segment (start 136.162008 73.7) (end 136.631371 73.7) (width 0.4) (layer "B.Cu") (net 3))
 (segment (start 140.3 70.031371) (end 140.3 65.21) (width 0.4) (layer "B.Cu") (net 3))
 (segment (start 136.631371 73.7) (end 140.3 70.031371) (width 0.4) (layer "B.Cu") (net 3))
 (segment (start 139.04 65.21) (end 136.3 67.95) (width 0.4) (layer "B.Cu") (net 3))
 (segment (start 136.0005 67.95) (end 136.0005 69.2495) (width 0.4) (layer "B.Cu") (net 3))
 (segment (start 136.3 67.95) (end 136.0005 67.95) (width 0.4) (layer "B.Cu") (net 3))
 (segment (start 136 69.25) (end 131.05 69.25) (width 0.4) (layer "B.Cu") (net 3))
 (segment (start 140.3 65.21) (end 139.04 65.21) (width 0.4) (layer "B.Cu") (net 3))
 (segment (start 130.9875 76.35) (end 130.55 75.9125) (width 0.25) (layer "F.Cu") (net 13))
 (segment (start 128.89 70.29) (end 127.9 70.29) (width 0.2) (layer "F.Cu") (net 13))
 (segment (start 132.75 71.95) (end 130.55 71.95) (width 0.2) (layer "F.Cu") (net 13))
 (segment (start 130.55 71.95) (end 128.89 70.29) (width 0.2) (layer "F.Cu") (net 13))
 (segment (start 130.55 75.9125) (end 130.55 71.95) (width 0.25) (layer "F.Cu") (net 13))
 (segment (start 126.5 69.7) (end 127.2 69) (width 0.2) (layer "F.Cu") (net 12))
 (segment (start 130.45 67.6) (end 129.05 69) (width 0.25) (layer "F.Cu") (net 12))
 (segment (start 126.93 72.83) (end 126.5 72.4) (width 0.2) (layer "F.Cu") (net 12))
 (segment (start 126.5 72.4) (end 126.5 69.7) (width 0.2) (layer "F.Cu") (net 12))
 (segment (start 129.05 69) (end 131.6 71.55) (width 0.2) (layer "F.Cu") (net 12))
 (segment (start 131.6 71.55) (end 132.75 71.55) (width 0.2) (layer "F.Cu") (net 12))
 (segment (start 127.2 69) (end 129.05 69) (width 0.2) (layer "F.Cu") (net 12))
 (segment (start 130.45 66.3625) (end 130.45 67.6) (width 0.25) (layer "F.Cu") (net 12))
 (segment (start 127.9 72.83) (end 126.93 72.83) (width 0.2) (layer "F.Cu") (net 12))
 (segment (start 137.8 74.7625) (end 138.9375 74.7625) (width 0.3) (layer "F.Cu") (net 2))
 (segment (start 133.25 68.7) (end 133.25 69.45) (width 0.2) (layer "F.Cu") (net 2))
 (segment (start 134.55 65.9375) (end 135.05 65.4375) (width 0.4) (layer "F.Cu") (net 2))
 (segment (start 133 68.4) (end 132.7 68.7) (width 0.4) (layer "F.Cu") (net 2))
 (segment (start 136.901744 71.15) (end 137.475872 71.724128) (width 0.2) (layer "F.Cu") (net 2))
 (segment (start 135.05 65.4375) (end 135.05 64.25) (width 0.4) (layer "F.Cu") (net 2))
 (segment (start 133 66.55) (end 133 68.4) (width 0.4) (layer "F.Cu") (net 2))
 (segment (start 131.85 69.95) (end 131.85 69.55) (width 0.4) (layer "F.Cu") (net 2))
 (segment (start 139.5 74.2) (end 139.5 72.75) (width 0.3) (layer "F.Cu") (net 2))
 (segment (start 138.9375 74.7625) (end 139.5 74.2) (width 0.3) (layer "F.Cu") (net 2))
 (segment (start 139.5 72.75) (end 138.474128 71.724128) (width 0.3) (layer "F.Cu") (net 2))
 (segment (start 138.3 65.35) (end 140.98 62.67) (width 0.4) (layer "F.Cu") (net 2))
 (segment (start 140.98 62.67) (end 143.075 62.67) (width 0.4) (layer "F.Cu") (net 2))
 (segment (start 131.85 69.55) (end 132.7 68.7) (width 0.4) (layer "F.Cu") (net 2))
 (segment (start 132.25 70.35) (end 132.75 70.35) (width 0.2) (layer "F.Cu") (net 2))
 (segment (start 135.75 71.15) (end 136.901744 71.15) (width 0.2) (layer "F.Cu") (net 2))
 (segment (start 134.55 65.9375) (end 133.6125 65.9375) (width 0.4) (layer "F.Cu") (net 2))
 (segment (start 133.6125 65.9375) (end 133 66.55) (width 0.4) (layer "F.Cu") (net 2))
 (segment (start 138.3 68.7375) (end 138.3 65.35) (width 0.4) (layer "F.Cu") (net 2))
 (segment (start 131.85 69.95) (end 132.25 70.35) (width 0.2) (layer "F.Cu") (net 2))
 (segment (start 133.25 68.7) (end 132.7 68.7) (width 0.2) (layer "F.Cu") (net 2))
 (segment (start 138.474128 71.724128) (end 137.475872 71.724128) (width 0.3) (layer "F.Cu") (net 2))
 (via (at 131.85 69.95) (size 0.6) (drill 0.3) (layers "F.Cu" "B.Cu") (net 2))
 (via (at 135.05 64.25) (size 0.6) (drill 0.3) (layers "F.Cu" "B.Cu") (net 2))
 (via (at 137.475872 71.724128) (size 0.8) (drill 0.4) (layers "F.Cu" "B.Cu") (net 2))
 (segment (start 136.63 62.67) (end 135.05 64.25) (width 0.4) (layer "B.Cu") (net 2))
 (segment (start 143.075 62.67) (end 136.63 62.67) (width 0.4) (layer "B.Cu") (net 2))
 (segment (start 131.8 70) (end 131.8 72.6) (width 0.4) (layer "B.Cu") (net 2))
 (segment (start 131.8 72.6) (end 136.6 72.6) (width 0.4) (layer "B.Cu") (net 2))
 (segment (start 131.85 69.95) (end 131.8 70) (width 0.4) (layer "B.Cu") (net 2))
 (segment (start 136.6 72.6) (end 137.475872 71.724128) (width 0.4) (layer "B.Cu") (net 2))
 (segment (start 138.0125 70.75) (end 138.3 70.4625) (width 0.2) (layer "F.Cu") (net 9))
 (segment (start 135.75 70.75) (end 138.0125 70.75) (width 0.2) (layer "F.Cu") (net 9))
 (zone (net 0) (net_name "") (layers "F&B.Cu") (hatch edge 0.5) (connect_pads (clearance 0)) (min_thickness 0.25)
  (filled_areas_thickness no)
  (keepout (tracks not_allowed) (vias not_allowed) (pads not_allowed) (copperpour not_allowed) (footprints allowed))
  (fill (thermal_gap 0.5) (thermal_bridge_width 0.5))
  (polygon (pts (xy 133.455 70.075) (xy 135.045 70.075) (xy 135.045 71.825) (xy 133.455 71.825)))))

